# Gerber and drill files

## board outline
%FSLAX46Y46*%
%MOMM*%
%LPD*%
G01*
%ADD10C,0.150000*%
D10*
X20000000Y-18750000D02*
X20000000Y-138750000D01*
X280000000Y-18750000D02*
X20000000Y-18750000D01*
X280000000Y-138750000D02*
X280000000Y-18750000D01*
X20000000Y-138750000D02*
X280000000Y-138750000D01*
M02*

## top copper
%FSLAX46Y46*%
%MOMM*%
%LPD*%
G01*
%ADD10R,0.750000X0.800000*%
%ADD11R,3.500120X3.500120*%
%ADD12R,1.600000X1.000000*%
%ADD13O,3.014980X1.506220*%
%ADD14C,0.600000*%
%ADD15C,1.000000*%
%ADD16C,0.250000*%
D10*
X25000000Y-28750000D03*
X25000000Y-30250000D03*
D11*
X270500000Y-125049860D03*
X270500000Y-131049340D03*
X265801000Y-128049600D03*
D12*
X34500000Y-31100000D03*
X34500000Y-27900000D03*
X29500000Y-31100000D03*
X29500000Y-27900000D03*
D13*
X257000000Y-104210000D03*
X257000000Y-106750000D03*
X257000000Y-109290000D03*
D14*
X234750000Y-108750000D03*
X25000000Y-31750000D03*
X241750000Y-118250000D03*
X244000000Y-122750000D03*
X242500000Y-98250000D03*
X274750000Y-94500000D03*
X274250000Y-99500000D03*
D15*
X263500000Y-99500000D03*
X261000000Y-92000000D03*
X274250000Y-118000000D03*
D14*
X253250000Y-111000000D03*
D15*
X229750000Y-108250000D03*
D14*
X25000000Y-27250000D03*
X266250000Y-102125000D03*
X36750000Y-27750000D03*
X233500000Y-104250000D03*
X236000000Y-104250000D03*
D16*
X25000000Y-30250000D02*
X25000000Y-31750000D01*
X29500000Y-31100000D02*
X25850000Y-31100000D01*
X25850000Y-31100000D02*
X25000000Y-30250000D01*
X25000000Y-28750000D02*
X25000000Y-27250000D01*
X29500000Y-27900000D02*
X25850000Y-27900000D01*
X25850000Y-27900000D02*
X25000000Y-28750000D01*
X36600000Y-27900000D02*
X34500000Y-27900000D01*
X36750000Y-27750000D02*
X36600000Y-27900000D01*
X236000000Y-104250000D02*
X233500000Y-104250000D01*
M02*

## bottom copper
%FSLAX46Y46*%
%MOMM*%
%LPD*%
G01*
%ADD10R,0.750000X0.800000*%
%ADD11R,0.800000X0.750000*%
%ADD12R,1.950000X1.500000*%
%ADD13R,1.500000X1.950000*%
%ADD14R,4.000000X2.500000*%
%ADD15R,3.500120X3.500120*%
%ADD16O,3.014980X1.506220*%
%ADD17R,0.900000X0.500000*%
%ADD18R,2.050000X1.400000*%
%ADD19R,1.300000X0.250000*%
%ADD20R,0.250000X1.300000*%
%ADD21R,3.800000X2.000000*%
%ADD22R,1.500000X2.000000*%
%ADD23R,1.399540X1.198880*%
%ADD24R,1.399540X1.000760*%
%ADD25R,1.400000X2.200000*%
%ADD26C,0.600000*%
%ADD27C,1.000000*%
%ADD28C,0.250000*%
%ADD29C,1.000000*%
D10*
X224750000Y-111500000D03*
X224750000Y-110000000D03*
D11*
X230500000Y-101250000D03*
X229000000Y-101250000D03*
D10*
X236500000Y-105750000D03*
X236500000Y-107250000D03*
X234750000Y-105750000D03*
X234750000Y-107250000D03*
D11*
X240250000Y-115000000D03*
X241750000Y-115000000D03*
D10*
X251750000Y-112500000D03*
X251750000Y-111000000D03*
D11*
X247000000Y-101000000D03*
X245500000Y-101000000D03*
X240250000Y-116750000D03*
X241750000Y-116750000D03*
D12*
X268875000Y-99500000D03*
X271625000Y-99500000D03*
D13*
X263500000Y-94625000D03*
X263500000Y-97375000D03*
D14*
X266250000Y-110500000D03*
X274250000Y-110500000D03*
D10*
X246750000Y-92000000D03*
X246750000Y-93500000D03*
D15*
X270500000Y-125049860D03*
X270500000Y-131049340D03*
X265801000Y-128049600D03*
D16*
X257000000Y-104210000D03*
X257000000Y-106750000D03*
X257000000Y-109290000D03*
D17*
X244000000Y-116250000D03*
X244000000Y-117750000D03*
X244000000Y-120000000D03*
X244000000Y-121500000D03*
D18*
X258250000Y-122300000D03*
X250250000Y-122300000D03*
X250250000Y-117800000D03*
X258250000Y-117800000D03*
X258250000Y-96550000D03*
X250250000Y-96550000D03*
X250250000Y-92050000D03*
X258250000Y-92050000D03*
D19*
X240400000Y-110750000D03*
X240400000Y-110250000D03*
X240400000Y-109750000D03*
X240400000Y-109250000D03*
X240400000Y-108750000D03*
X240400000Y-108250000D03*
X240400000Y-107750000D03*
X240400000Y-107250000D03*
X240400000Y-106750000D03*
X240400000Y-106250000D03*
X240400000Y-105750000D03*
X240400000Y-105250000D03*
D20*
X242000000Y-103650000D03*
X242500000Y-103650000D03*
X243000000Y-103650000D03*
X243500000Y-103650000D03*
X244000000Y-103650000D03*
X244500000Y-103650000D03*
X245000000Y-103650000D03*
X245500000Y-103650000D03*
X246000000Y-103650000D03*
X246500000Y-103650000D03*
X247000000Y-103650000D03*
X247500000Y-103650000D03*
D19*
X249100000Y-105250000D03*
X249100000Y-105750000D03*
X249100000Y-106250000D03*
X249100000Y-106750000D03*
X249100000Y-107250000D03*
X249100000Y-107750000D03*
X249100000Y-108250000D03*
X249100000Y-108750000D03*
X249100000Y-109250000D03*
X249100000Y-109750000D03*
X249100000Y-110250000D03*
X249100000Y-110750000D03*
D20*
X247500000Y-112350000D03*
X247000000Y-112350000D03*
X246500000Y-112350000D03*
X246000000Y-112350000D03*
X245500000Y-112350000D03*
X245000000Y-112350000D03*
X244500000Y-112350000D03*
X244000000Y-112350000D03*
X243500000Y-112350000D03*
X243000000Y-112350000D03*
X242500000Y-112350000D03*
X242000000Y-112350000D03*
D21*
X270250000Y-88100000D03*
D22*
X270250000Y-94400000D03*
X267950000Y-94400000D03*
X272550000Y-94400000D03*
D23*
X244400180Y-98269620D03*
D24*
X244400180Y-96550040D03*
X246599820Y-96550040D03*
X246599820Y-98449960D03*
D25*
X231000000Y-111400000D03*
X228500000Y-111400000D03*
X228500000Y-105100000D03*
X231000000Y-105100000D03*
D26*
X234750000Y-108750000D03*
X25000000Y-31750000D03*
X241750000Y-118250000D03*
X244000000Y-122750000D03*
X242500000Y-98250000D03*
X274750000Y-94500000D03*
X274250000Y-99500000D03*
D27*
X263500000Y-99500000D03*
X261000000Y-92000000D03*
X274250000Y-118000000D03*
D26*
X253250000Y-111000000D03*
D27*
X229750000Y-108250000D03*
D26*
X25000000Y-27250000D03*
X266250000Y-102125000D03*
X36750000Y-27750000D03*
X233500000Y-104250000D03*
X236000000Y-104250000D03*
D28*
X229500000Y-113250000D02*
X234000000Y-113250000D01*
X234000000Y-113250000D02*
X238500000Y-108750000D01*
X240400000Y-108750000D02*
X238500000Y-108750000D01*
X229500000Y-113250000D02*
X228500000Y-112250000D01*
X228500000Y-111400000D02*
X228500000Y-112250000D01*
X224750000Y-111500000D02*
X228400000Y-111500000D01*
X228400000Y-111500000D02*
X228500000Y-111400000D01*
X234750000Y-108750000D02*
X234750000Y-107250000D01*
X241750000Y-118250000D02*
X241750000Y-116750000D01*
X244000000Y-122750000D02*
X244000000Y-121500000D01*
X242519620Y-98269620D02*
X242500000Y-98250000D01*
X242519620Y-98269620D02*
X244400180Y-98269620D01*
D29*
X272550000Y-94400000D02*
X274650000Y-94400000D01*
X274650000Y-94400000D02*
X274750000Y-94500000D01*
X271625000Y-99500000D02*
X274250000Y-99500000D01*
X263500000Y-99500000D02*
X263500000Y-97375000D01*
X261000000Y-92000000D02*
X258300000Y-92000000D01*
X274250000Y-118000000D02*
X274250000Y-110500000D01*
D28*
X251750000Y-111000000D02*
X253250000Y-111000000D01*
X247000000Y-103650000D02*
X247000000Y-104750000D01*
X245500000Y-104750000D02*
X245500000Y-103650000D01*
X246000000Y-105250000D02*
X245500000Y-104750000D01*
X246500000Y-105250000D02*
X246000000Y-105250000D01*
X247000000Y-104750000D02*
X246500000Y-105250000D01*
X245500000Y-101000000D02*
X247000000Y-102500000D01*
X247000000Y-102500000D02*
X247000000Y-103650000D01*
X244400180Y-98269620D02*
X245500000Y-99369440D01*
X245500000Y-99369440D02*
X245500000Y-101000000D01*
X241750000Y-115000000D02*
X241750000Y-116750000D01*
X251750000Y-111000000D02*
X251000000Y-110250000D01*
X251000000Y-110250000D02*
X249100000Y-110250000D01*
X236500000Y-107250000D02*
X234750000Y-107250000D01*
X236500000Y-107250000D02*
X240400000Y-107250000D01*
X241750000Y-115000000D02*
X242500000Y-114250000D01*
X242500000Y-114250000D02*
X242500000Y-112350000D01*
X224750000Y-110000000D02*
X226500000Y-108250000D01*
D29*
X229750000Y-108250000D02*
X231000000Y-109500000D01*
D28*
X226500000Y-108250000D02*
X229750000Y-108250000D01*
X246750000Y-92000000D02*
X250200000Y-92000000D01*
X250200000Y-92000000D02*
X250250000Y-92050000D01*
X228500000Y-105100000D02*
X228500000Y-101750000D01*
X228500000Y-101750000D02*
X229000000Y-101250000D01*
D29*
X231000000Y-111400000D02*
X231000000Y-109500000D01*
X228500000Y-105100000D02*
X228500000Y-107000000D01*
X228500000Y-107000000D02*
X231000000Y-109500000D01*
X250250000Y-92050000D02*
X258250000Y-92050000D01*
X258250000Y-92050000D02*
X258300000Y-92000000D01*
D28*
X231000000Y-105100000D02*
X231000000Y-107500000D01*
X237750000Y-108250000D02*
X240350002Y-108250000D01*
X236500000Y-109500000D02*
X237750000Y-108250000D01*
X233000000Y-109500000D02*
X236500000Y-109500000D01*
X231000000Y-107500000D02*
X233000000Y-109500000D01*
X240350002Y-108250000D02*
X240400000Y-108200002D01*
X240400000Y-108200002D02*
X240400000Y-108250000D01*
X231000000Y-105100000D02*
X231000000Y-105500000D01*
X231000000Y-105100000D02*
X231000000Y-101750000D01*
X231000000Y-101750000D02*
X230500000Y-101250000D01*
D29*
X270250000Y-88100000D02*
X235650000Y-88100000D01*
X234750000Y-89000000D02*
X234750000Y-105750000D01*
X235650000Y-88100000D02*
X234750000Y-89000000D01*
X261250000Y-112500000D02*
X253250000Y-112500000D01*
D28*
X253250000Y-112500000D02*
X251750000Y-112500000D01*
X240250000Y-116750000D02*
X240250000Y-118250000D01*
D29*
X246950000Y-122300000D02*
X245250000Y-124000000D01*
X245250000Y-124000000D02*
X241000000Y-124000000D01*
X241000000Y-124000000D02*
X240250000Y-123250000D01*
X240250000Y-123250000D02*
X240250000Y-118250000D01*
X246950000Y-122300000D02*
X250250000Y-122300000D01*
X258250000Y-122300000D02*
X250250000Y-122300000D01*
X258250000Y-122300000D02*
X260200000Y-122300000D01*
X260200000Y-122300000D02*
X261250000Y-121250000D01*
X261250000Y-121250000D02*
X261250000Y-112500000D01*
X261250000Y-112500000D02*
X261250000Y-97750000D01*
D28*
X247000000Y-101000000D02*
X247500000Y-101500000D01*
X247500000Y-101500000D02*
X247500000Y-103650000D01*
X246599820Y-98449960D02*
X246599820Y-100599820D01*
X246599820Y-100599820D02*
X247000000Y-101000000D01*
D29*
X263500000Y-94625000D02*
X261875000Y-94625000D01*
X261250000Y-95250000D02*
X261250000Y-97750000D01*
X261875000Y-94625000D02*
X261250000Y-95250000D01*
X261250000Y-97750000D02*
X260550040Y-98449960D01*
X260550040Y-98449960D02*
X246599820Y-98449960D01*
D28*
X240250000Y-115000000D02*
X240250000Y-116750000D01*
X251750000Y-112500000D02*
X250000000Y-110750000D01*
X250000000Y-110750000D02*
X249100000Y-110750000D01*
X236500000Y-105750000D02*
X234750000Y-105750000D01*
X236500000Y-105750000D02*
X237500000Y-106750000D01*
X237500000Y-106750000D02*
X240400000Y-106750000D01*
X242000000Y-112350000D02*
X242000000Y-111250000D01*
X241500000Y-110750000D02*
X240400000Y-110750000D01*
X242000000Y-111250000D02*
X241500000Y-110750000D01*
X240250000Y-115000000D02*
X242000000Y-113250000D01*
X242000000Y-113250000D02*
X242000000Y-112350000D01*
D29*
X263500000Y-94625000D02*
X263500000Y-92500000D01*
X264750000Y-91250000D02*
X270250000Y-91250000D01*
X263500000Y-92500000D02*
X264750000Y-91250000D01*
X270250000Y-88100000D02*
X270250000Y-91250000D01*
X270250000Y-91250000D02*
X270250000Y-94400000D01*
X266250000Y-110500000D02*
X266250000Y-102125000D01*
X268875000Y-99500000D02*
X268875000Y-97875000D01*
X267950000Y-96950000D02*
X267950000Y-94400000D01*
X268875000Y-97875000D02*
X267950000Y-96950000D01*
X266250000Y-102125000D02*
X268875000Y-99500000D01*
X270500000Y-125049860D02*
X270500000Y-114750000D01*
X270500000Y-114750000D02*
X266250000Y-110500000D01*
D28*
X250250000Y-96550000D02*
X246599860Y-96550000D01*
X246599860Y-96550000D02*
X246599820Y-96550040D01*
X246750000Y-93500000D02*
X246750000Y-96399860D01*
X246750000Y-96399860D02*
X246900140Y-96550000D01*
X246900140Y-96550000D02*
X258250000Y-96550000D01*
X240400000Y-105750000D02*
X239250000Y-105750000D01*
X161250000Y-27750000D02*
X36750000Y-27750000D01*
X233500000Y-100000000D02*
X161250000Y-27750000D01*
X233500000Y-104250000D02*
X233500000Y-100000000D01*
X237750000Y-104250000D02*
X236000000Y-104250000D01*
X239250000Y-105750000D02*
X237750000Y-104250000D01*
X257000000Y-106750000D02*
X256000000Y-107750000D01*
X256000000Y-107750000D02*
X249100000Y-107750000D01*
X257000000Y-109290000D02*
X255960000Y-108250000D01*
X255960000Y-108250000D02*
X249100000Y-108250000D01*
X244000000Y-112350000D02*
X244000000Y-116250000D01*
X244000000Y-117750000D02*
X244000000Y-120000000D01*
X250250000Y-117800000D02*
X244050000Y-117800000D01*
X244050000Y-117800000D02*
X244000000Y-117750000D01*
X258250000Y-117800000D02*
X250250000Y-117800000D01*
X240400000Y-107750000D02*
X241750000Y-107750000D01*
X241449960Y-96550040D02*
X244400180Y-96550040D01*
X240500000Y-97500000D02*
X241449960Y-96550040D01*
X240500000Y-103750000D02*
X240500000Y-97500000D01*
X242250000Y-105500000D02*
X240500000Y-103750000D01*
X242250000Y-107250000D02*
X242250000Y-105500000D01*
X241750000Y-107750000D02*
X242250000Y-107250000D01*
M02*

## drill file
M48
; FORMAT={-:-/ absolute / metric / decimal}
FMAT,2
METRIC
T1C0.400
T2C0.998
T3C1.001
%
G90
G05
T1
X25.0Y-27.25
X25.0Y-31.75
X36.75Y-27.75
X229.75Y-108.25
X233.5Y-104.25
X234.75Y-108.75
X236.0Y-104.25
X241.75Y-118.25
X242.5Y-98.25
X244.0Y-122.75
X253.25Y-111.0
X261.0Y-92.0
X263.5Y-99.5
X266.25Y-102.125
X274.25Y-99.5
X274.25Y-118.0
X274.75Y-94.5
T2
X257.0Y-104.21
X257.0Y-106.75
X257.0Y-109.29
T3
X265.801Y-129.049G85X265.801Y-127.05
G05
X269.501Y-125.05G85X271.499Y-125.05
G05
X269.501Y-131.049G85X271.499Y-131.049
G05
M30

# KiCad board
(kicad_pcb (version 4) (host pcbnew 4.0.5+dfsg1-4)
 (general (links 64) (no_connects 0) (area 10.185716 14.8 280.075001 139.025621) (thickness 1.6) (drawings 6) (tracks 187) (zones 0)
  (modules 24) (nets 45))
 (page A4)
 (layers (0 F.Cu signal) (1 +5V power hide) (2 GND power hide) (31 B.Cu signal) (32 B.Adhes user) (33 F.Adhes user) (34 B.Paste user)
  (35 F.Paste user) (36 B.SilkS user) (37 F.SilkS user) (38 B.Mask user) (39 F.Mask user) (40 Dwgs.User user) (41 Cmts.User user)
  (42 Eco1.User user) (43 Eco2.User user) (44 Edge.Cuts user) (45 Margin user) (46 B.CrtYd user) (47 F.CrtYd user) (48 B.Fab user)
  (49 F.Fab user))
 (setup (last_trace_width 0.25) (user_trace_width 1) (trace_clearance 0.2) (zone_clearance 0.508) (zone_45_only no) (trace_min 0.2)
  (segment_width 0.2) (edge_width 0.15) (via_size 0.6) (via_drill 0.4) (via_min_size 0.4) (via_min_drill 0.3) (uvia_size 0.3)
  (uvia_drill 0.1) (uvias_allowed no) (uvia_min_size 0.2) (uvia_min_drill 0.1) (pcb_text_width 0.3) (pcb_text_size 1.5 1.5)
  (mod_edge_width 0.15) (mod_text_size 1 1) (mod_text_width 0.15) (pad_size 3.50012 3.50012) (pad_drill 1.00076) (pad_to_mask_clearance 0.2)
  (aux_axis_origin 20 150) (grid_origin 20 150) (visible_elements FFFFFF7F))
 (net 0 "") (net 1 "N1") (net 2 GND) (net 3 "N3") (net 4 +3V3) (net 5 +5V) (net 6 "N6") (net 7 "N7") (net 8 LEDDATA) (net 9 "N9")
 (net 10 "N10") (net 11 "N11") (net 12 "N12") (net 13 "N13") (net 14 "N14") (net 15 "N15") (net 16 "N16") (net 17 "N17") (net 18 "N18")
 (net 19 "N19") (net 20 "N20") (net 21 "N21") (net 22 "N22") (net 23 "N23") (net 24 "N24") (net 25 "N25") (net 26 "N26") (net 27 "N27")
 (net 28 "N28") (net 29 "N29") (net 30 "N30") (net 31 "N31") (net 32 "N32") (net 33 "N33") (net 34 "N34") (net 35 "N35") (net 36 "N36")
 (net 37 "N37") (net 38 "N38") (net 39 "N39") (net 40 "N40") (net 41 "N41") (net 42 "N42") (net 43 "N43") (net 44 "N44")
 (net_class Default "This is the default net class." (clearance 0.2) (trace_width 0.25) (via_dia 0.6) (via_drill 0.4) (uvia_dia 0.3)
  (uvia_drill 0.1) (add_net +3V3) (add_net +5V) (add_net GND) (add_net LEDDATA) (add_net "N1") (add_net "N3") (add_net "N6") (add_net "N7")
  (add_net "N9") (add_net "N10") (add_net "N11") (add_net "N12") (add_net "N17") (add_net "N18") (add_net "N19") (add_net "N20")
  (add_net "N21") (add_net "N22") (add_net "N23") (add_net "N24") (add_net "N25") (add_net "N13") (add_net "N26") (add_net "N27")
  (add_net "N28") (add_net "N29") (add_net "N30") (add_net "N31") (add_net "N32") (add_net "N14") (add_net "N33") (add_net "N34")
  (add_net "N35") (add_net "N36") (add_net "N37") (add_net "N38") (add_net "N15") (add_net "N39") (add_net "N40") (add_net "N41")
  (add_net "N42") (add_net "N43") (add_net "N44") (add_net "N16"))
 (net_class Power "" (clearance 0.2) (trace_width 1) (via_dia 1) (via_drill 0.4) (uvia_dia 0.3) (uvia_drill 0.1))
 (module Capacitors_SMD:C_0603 (layer B.Cu) (at 224.75 110.75 90)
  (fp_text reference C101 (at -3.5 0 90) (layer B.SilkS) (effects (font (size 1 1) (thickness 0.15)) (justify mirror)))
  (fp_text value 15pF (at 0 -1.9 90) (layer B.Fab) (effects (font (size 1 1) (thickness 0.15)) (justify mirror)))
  (pad 1 smd rect (at -0.75 0 90) (size 0.8 0.75) (layers B.Cu B.Paste B.Mask) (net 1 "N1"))
  (pad 2 smd rect (at 0.75 0 90) (size 0.8 0.75) (layers B.Cu B.Paste B.Mask) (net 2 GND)))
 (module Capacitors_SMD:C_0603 (layer B.Cu) (at 229.75 101.25 180)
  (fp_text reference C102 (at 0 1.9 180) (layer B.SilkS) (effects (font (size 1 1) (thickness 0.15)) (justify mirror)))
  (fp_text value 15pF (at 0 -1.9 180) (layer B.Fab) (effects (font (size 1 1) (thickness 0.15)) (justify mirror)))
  (pad 1 smd rect (at -0.75 0 180) (size 0.8 0.75) (layers B.Cu B.Paste B.Mask) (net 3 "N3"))
  (pad 2 smd rect (at 0.75 0 180) (size 0.8 0.75) (layers B.Cu B.Paste B.Mask) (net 2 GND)))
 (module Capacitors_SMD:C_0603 (layer B.Cu) (at 236.5 106.5 270)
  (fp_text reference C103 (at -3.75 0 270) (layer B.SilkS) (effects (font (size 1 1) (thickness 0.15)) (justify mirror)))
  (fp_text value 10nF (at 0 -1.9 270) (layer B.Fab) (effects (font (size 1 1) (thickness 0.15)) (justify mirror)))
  (pad 1 smd rect (at -0.75 0 270) (size 0.8 0.75) (layers B.Cu B.Paste B.Mask) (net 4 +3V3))
  (pad 2 smd rect (at 0.75 0 270) (size 0.8 0.75) (layers B.Cu B.Paste B.Mask) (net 2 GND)))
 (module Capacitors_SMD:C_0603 (layer B.Cu) (at 234.75 106.5 270)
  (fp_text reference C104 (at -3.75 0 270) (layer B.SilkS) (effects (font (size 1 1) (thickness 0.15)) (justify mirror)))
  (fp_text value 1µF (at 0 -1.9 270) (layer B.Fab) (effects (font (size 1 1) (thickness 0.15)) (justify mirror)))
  (pad 1 smd rect (at -0.75 0 270) (size 0.8 0.75) (layers B.Cu B.Paste B.Mask) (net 4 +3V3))
  (pad 2 smd rect (at 0.75 0 270) (size 0.8 0.75) (layers B.Cu B.Paste B.Mask) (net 2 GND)))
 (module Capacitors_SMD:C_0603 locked (layer B.Cu) (at 241 115)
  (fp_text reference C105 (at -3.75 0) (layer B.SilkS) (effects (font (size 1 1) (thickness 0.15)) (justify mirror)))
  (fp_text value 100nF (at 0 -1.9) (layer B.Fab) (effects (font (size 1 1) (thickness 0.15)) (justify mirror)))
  (pad 1 smd rect (at -0.75 0) (size 0.8 0.75) (layers B.Cu B.Paste B.Mask) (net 4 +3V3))
  (pad 2 smd rect (at 0.75 0) (size 0.8 0.75) (layers B.Cu B.Paste B.Mask) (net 2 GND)))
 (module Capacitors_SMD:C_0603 (layer B.Cu) (at 251.75 111.75 90)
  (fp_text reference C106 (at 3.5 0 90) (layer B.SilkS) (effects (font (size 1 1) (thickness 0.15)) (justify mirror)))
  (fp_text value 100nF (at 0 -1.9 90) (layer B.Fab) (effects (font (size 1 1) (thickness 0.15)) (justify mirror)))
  (pad 1 smd rect (at -0.75 0 90) (size 0.8 0.75) (layers B.Cu B.Paste B.Mask) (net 4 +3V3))
  (pad 2 smd rect (at 0.75 0 90) (size 0.8 0.75) (layers B.Cu B.Paste B.Mask) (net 2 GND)))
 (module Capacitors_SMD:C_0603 (layer B.Cu) (at 246.25 101 180)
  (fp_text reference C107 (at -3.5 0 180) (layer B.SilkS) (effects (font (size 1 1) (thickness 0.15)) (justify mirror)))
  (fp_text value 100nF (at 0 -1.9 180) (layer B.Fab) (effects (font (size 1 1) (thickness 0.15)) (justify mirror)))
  (pad 1 smd rect (at -0.75 0 180) (size 0.8 0.75) (layers B.Cu B.Paste B.Mask) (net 4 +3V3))
  (pad 2 smd rect (at 0.75 0 180) (size 0.8 0.75) (layers B.Cu B.Paste B.Mask) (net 2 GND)))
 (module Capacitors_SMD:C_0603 (layer B.Cu) (at 241 116.75)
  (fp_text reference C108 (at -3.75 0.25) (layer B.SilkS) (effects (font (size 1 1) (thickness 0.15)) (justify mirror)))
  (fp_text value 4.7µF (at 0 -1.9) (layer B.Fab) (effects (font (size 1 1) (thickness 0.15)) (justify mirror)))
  (pad 1 smd rect (at -0.75 0) (size 0.8 0.75) (layers B.Cu B.Paste B.Mask) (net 4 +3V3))
  (pad 2 smd rect (at 0.75 0) (size 0.8 0.75) (layers B.Cu B.Paste B.Mask) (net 2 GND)))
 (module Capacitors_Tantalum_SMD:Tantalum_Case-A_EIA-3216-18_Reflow (layer B.Cu) (at 270.25 99.5)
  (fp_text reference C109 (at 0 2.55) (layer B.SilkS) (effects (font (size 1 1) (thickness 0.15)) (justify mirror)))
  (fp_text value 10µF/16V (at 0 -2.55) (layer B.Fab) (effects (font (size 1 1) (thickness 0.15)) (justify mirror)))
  (pad 1 smd rect (at -1.375 0) (size 1.95 1.5) (layers B.Cu B.Paste B.Mask) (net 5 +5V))
  (pad 2 smd rect (at 1.375 0) (size 1.95 1.5) (layers B.Cu B.Paste B.Mask) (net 2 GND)))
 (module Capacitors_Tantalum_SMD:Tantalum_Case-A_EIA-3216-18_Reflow (layer B.Cu) (at 263.5 96 270)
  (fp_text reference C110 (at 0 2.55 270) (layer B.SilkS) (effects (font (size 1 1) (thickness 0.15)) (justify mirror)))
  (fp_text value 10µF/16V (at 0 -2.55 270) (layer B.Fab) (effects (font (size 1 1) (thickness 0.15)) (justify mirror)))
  (pad 1 smd rect (at -1.375 0 270) (size 1.95 1.5) (layers B.Cu B.Paste B.Mask) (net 4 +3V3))
  (pad 2 smd rect (at 1.375 0 270) (size 1.95 1.5) (layers B.Cu B.Paste B.Mask) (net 2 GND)))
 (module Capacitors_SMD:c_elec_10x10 (layer B.Cu) (at 270.25 110.5)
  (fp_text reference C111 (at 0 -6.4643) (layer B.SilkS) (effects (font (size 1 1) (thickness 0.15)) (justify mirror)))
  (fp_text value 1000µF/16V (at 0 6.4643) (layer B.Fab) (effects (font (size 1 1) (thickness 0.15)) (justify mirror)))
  (pad 1 smd rect (at -4 0 180) (size 4 2.5) (layers B.Cu B.Paste B.Mask) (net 5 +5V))
  (pad 2 smd rect (at 4 0 180) (size 4 2.5) (layers B.Cu B.Paste B.Mask) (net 2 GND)))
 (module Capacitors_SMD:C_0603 (layer B.Cu) (at 246.75 92.75 270)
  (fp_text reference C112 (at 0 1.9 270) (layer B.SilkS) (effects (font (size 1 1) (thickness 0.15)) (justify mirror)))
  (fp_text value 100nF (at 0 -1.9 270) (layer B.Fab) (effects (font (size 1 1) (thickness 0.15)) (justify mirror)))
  (pad 1 smd rect (at -0.75 0 270) (size 0.8 0.75) (layers B.Cu B.Paste B.Mask) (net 2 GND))
  (pad 2 smd rect (at 0.75 0 270) (size 0.8 0.75) (layers B.Cu B.Paste B.Mask) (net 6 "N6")))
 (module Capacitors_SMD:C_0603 (layer F.Cu) (at 25 29.5 270)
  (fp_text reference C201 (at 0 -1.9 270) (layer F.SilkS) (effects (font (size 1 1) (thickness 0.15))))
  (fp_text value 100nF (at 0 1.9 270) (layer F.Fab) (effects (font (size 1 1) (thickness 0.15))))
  (pad 1 smd rect (at -0.75 0 270) (size 0.8 0.75) (layers F.Cu F.Paste F.Mask) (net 5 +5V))
  (pad 2 smd rect (at 0.75 0 270) (size 0.8 0.75) (layers F.Cu F.Paste F.Mask) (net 2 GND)))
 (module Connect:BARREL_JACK (layer B.Cu) (at 270.5 131.25 90)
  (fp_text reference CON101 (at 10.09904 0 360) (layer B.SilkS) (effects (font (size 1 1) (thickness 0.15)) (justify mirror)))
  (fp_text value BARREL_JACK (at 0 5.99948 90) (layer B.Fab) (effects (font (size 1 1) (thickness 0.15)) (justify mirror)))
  (pad 1 thru_hole rect (at 6.20014 0 90) (size 3.50012 3.50012) (drill oval 1.00076 2.99974) (layers *.Cu *.Mask) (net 5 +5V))
  (pad 2 thru_hole rect (at 0.20066 0 90) (size 3.50012 3.50012) (drill oval 1.00076 2.99974) (layers *.Cu *.Mask) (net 2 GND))
  (pad 3 thru_hole rect (at 3.2004 -4.699 90) (size 3.50012 3.50012) (drill oval 2.99974 1.00076) (layers *.Cu *.Mask) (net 2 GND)))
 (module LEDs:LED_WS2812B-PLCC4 (layer F.Cu) (at 32 29.5)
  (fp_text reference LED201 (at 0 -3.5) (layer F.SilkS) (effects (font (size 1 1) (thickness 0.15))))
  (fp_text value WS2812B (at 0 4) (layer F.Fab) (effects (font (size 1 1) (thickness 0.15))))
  (pad 3 smd rect (at 2.5 1.6) (size 1.6 1) (layers F.Cu F.Paste F.Mask) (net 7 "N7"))
  (pad 4 smd rect (at 2.5 -1.6) (size 1.6 1) (layers F.Cu F.Paste F.Mask) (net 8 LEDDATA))
  (pad 2 smd rect (at -2.5 1.6) (size 1.6 1) (layers F.Cu F.Paste F.Mask) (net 2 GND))
  (pad 1 smd rect (at -2.5 -1.6) (size 1.6 1) (layers F.Cu F.Paste F.Mask) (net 5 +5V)))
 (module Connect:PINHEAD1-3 (layer B.Cu) (at 257 106.75 270)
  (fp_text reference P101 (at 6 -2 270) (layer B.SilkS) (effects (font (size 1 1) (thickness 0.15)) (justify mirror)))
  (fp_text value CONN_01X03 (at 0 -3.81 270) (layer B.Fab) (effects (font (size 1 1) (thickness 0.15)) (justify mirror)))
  (pad 1 thru_hole oval (at -2.54 0 270) (size 1.50622 3.01498) (drill 0.99822) (layers *.Cu *.Mask) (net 2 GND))
  (pad 2 thru_hole oval (at 0 0 270) (size 1.50622 3.01498) (drill 0.99822) (layers *.Cu *.Mask) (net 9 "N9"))
  (pad 3 thru_hole oval (at 2.54 0 270) (size 1.50622 3.01498) (drill 0.99822) (layers *.Cu *.Mask) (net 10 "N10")))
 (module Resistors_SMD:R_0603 (layer B.Cu) (at 244 117 270)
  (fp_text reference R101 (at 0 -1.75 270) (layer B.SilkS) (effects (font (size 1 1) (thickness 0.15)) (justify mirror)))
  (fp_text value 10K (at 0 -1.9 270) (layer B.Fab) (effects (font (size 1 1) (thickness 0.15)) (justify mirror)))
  (pad 1 smd rect (at -0.75 0 270) (size 0.5 0.9) (layers B.Cu B.Paste B.Mask) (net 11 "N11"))
  (pad 2 smd rect (at 0.75 0 270) (size 0.5 0.9) (layers B.Cu B.Paste B.Mask) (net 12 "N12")))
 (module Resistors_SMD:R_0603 (layer B.Cu) (at 244 120.75 270)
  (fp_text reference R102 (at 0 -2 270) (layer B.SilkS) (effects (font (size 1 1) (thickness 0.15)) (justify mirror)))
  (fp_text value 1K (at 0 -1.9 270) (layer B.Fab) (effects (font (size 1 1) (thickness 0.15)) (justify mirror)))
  (pad 1 smd rect (at -0.75 0 270) (size 0.5 0.9) (layers B.Cu B.Paste B.Mask) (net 12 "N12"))
  (pad 2 smd rect (at 0.75 0 270) (size 0.5 0.9) (layers B.Cu B.Paste B.Mask) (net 2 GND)))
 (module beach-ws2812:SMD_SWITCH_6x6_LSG (layer B.Cu) (at 249.25 123)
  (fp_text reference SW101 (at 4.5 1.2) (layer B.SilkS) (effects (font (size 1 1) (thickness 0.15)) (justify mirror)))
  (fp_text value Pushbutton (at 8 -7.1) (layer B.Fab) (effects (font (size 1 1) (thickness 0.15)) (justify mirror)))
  (pad 2 smd rect (at 9 -0.7) (size 2.05 1.4) (layers B.Cu B.Paste B.Mask) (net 4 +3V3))
  (pad 1 smd rect (at 1 -0.7) (size 2.05 1.4) (layers B.Cu B.Paste B.Mask) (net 4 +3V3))
  (pad 3 smd rect (at 1 -5.2) (size 2.05 1.4) (layers B.Cu B.Paste B.Mask) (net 12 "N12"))
  (pad 4 smd rect (at 9 -5.2) (size 2.05 1.4) (layers B.Cu B.Paste B.Mask) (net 12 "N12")))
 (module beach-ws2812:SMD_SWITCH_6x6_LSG (layer B.Cu) (at 249.25 97.25)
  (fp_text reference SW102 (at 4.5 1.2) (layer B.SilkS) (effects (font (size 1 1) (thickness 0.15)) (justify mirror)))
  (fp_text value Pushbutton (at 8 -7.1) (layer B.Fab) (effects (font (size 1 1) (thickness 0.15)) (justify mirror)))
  (pad 2 smd rect (at 9 -0.7) (size 2.05 1.4) (layers B.Cu B.Paste B.Mask) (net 6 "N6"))
  (pad 1 smd rect (at 1 -0.7) (size 2.05 1.4) (layers B.Cu B.Paste B.Mask) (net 6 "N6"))
  (pad 3 smd rect (at 1 -5.2) (size 2.05 1.4) (layers B.Cu B.Paste B.Mask) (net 2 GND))
  (pad 4 smd rect (at 9 -5.2) (size 2.05 1.4) (layers B.Cu B.Paste B.Mask) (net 2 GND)))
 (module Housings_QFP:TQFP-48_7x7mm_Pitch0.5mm (layer B.Cu) (at 244.75 108)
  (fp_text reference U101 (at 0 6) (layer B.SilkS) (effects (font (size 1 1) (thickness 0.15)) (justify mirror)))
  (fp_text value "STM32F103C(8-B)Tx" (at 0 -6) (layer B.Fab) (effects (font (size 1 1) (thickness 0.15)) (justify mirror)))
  (pad 1 smd rect (at -4.35 2.75) (size 1.3 0.25) (layers B.Cu B.Paste B.Mask) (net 4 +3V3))
  (pad 2 smd rect (at -4.35 2.25) (size 1.3 0.25) (layers B.Cu B.Paste B.Mask) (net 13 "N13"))
  (pad 3 smd rect (at -4.35 1.75) (size 1.3 0.25) (layers B.Cu B.Paste B.Mask) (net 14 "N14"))
  (pad 4 smd rect (at -4.35 1.25) (size 1.3 0.25) (layers B.Cu B.Paste B.Mask) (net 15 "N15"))
  (pad 5 smd rect (at -4.35 0.75) (size 1.3 0.25) (layers B.Cu B.Paste B.Mask) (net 1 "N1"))
  (pad 6 smd rect (at -4.35 0.25) (size 1.3 0.25) (layers B.Cu B.Paste B.Mask) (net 3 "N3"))
  (pad 7 smd rect (at -4.35 -0.25) (size 1.3 0.25) (layers B.Cu B.Paste B.Mask) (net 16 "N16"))
  (pad 8 smd rect (at -4.35 -0.75) (size 1.3 0.25) (layers B.Cu B.Paste B.Mask) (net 2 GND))
  (pad 9 smd rect (at -4.35 -1.25) (size 1.3 0.25) (layers B.Cu B.Paste B.Mask) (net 4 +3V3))
  (pad 10 smd rect (at -4.35 -1.75) (size 1.3 0.25) (layers B.Cu B.Paste B.Mask) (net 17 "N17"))
  (pad 11 smd rect (at -4.35 -2.25) (size 1.3 0.25) (layers B.Cu B.Paste B.Mask) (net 8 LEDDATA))
  (pad 12 smd rect (at -4.35 -2.75) (size 1.3 0.25) (layers B.Cu B.Paste B.Mask) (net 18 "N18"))
  (pad 13 smd rect (at -2.75 -4.35 270) (size 1.3 0.25) (layers B.Cu B.Paste B.Mask) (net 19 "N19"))
  (pad 14 smd rect (at -2.25 -4.35 270) (size 1.3 0.25) (layers B.Cu B.Paste B.Mask) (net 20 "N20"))
  (pad 15 smd rect (at -1.75 -4.35 270) (size 1.3 0.25) (layers B.Cu B.Paste B.Mask) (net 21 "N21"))
  (pad 16 smd rect (at -1.25 -4.35 270) (size 1.3 0.25) (layers B.Cu B.Paste B.Mask) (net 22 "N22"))
  (pad 17 smd rect (at -0.75 -4.35 270) (size 1.3 0.25) (layers B.Cu B.Paste B.Mask) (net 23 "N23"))
  (pad 18 smd rect (at -0.25 -4.35 270) (size 1.3 0.25) (layers B.Cu B.Paste B.Mask) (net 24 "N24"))
  (pad 19 smd rect (at 0.25 -4.35 270) (size 1.3 0.25) (layers B.Cu B.Paste B.Mask) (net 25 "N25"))
  (pad 20 smd rect (at 0.75 -4.35 270) (size 1.3 0.25) (layers B.Cu B.Paste B.Mask) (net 2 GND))
  (pad 21 smd rect (at 1.25 -4.35 270) (size 1.3 0.25) (layers B.Cu B.Paste B.Mask) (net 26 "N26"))
  (pad 22 smd rect (at 1.75 -4.35 270) (size 1.3 0.25) (layers B.Cu B.Paste B.Mask) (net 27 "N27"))
  (pad 23 smd rect (at 2.25 -4.35 270) (size 1.3 0.25) (layers B.Cu B.Paste B.Mask) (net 2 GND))
  (pad 24 smd rect (at 2.75 -4.35 270) (size 1.3 0.25) (layers B.Cu B.Paste B.Mask) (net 4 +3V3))
  (pad 25 smd rect (at 4.35 -2.75) (size 1.3 0.25) (layers B.Cu B.Paste B.Mask) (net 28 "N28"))
  (pad 26 smd rect (at 4.35 -2.25) (size 1.3 0.25) (layers B.Cu B.Paste B.Mask) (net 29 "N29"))
  (pad 27 smd rect (at 4.35 -1.75) (size 1.3 0.25) (layers B.Cu B.Paste B.Mask) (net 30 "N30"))
  (pad 28 smd rect (at 4.35 -1.25) (size 1.3 0.25) (layers B.Cu B.Paste B.Mask) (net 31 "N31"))
  (pad 29 smd rect (at 4.35 -0.75) (size 1.3 0.25) (layers B.Cu B.Paste B.Mask) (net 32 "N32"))
  (pad 30 smd rect (at 4.35 -0.25) (size 1.3 0.25) (layers B.Cu B.Paste B.Mask) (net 9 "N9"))
  (pad 31 smd rect (at 4.35 0.25) (size 1.3 0.25) (layers B.Cu B.Paste B.Mask) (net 10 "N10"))
  (pad 32 smd rect (at 4.35 0.75) (size 1.3 0.25) (layers B.Cu B.Paste B.Mask) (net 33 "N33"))
  (pad 33 smd rect (at 4.35 1.25) (size 1.3 0.25) (layers B.Cu B.Paste B.Mask) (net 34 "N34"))
  (pad 34 smd rect (at 4.35 1.75) (size 1.3 0.25) (layers B.Cu B.Paste B.Mask) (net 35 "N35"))
  (pad 35 smd rect (at 4.35 2.25) (size 1.3 0.25) (layers B.Cu B.Paste B.Mask) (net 2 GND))
  (pad 36 smd rect (at 4.35 2.75) (size 1.3 0.25) (layers B.Cu B.Paste B.Mask) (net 4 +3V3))
  (pad 37 smd rect (at 2.75 4.35 270) (size 1.3 0.25) (layers B.Cu B.Paste B.Mask) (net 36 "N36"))
  (pad 38 smd rect (at 2.25 4.35 270) (size 1.3 0.25) (layers B.Cu B.Paste B.Mask) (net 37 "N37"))
  (pad 39 smd rect (at 1.75 4.35 270) (size 1.3 0.25) (layers B.Cu B.Paste B.Mask) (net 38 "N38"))
  (pad 40 smd rect (at 1.25 4.35 270) (size 1.3 0.25) (layers B.Cu B.Paste B.Mask) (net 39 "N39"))
  (pad 41 smd rect (at 0.75 4.35 270) (size 1.3 0.25) (layers B.Cu B.Paste B.Mask) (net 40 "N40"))
  (pad 42 smd rect (at 0.25 4.35 270) (size 1.3 0.25) (layers B.Cu B.Paste B.Mask) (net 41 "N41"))
  (pad 43 smd rect (at -0.25 4.35 270) (size 1.3 0.25) (layers B.Cu B.Paste B.Mask) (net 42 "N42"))
  (pad 44 smd rect (at -0.75 4.35 270) (size 1.3 0.25) (layers B.Cu B.Paste B.Mask) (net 11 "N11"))
  (pad 45 smd rect (at -1.25 4.35 270) (size 1.3 0.25) (layers B.Cu B.Paste B.Mask) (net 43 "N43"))
  (pad 46 smd rect (at -1.75 4.35 270) (size 1.3 0.25) (layers B.Cu B.Paste B.Mask) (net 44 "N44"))
  (pad 47 smd rect (at -2.25 4.35 270) (size 1.3 0.25) (layers B.Cu B.Paste B.Mask) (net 2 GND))
  (pad 48 smd rect (at -2.75 4.35 270) (size 1.3 0.25) (layers B.Cu B.Paste B.Mask) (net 4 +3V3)))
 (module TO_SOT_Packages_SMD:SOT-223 (layer B.Cu) (at 270.25 91.25 90)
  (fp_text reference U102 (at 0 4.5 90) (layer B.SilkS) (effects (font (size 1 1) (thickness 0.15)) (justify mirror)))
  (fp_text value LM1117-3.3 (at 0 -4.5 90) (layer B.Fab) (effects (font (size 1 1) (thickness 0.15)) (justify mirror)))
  (pad 4 smd rect (at 3.15 0 90) (size 2 3.8) (layers B.Cu B.Paste B.Mask) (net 4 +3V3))
  (pad 2 smd rect (at -3.15 0 90) (size 2 1.5) (layers B.Cu B.Paste B.Mask) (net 4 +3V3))
  (pad 3 smd rect (at -3.15 -2.3 90) (size 2 1.5) (layers B.Cu B.Paste B.Mask) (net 5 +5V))
  (pad 1 smd rect (at -3.15 2.3 90) (size 2 1.5) (layers B.Cu B.Paste B.Mask) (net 2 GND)))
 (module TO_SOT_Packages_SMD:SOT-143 (layer B.Cu) (at 245.5 97.5 90)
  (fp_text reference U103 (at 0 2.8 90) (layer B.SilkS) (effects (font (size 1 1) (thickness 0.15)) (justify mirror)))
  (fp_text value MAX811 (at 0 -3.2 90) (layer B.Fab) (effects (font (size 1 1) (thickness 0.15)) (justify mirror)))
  (pad 1 smd rect (at -0.76962 -1.09982 90) (size 1.19888 1.39954) (layers B.Cu B.Paste B.Mask) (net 2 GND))
  (pad 2 smd rect (at 0.94996 -1.09982 90) (size 1.00076 1.39954) (layers B.Cu B.Paste B.Mask) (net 16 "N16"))
  (pad 3 smd rect (at 0.94996 1.09982 90) (size 1.00076 1.39954) (layers B.Cu B.Paste B.Mask) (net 6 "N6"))
  (pad 4 smd rect (at -0.94996 1.09982 90) (size 1.00076 1.39954) (layers B.Cu B.Paste B.Mask) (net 4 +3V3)))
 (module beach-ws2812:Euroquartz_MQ (layer B.Cu) (at 229.75 108.25 90)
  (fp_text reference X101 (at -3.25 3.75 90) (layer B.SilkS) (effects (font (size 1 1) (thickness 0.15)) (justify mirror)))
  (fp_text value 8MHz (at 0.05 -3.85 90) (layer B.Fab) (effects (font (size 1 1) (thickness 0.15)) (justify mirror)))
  (pad 4 smd rect (at -3.15 1.25 90) (size 2.2 1.4) (layers B.Cu B.Paste B.Mask) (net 2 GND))
  (pad 1 smd rect (at -3.15 -1.25 90) (size 2.2 1.4) (layers B.Cu B.Paste B.Mask) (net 1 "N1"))
  (pad 2 smd rect (at 3.15 -1.25 90) (size 2.2 1.4) (layers B.Cu B.Paste B.Mask) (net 2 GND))
  (pad 3 smd rect (at 3.15 1.25 90) (size 2.2 1.4) (layers B.Cu B.Paste B.Mask) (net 3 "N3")))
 (gr_line (start 20 18.75) (end 20 138.75) (angle 90) (layer Edge.Cuts) (width 0.15))
 (gr_line (start 280 18.75) (end 20 18.75) (angle 90) (layer Edge.Cuts) (width 0.15))
 (gr_line (start 280 138.75) (end 280 18.75) (angle 90) (layer Edge.Cuts) (width 0.15))
 (gr_line (start 20 138.75) (end 280 138.75) (angle 90) (layer Edge.Cuts) (width 0.15))
 (segment (start 229.5 113.25) (end 234 113.25) (width 0.25) (layer B.Cu) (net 1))
 (segment (start 234 113.25) (end 238.5 108.75) (width 0.25) (layer B.Cu) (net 1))
 (segment (start 240.4 108.75) (end 238.5 108.75) (width 0.25) (layer B.Cu) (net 1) (status 10))
 (segment (start 229.5 113.25) (end 228.5 112.25) (width 0.25) (layer B.Cu) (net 1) (status 20))
 (segment (start 228.5 111.4) (end 228.5 112.25) (width 0.25) (layer B.Cu) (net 1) (status 30))
 (segment (start 224.75 111.5) (end 228.4 111.5) (width 0.25) (layer B.Cu) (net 1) (status 30))
 (segment (start 228.4 111.5) (end 228.5 111.4) (width 0.25) (layer B.Cu) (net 1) (status 30))
 (segment (start 235.5 108.75) (end 234.75 108.75) (width 0.25) (layer GND) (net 2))
 (via (at 234.75 108.75) (size 0.6) (drill 0.4) (layers F.Cu B.Cu) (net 2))
 (segment (start 234.75 108.75) (end 234.75 107.25) (width 0.25) (layer B.Cu) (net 2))
 (segment (start 25 30.25) (end 25 31.75) (width 0.25) (layer F.Cu) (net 2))
 (segment (start 25 31.75) (end 26 31.75) (width 0.25) (layer GND) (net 2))
 (via (at 25 31.75) (size 0.6) (drill 0.4) (layers F.Cu B.Cu) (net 2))
 (segment (start 29.5 31.1) (end 25.85 31.1) (width 0.25) (layer F.Cu) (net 2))
 (segment (start 25.85 31.1) (end 25 30.25) (width 0.25) (layer F.Cu) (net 2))
 (segment (start 241.75 119.5) (end 241.75 118.25) (width 1) (layer GND) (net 2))
 (via (at 241.75 118.25) (size 0.6) (drill 0.4) (layers F.Cu B.Cu) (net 2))
 (segment (start 241.75 118.25) (end 241.75 116.75) (width 0.25) (layer B.Cu) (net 2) (status 20))
 (segment (start 242.75 122.75) (end 244 122.75) (width 1) (layer GND) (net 2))
 (via (at 244 122.75) (size 0.6) (drill 0.4) (layers F.Cu B.Cu) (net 2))
 (segment (start 244 122.75) (end 244 121.5) (width 0.25) (layer B.Cu) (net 2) (status 20))
 (segment (start 241.25 98.25) (end 242.5 98.25) (width 1) (layer GND) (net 2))
 (segment (start 242.51962 98.26962) (end 242.5 98.25) (width 0.25) (layer B.Cu) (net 2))
 (via (at 242.5 98.25) (size 0.6) (drill 0.4) (layers F.Cu B.Cu) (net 2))
 (segment (start 242.51962 98.26962) (end 244.40018 98.26962) (width 0.25) (layer B.Cu) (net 2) (status 20))
 (segment (start 272.55 94.4) (end 274.65 94.4) (width 1) (layer B.Cu) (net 2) (status 10))
 (segment (start 274.75 94.5) (end 276 94.5) (width 1) (layer GND) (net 2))
 (via (at 274.75 94.5) (size 0.6) (drill 0.4) (layers F.Cu B.Cu) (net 2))
 (segment (start 274.65 94.4) (end 274.75 94.5) (width 1) (layer B.Cu) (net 2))
 (segment (start 271.625 99.5) (end 274.25 99.5) (width 1) (layer B.Cu) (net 2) (status 10))
 (segment (start 274.25 99.5) (end 275.75 99.5) (width 1) (layer GND) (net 2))
 (via (at 274.25 99.5) (size 0.6) (drill 0.4) (layers F.Cu B.Cu) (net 2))
 (segment (start 263.5 101.25) (end 263.5 99.5) (width 1) (layer GND) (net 2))
 (via (at 263.5 99.5) (size 1) (drill 0.4) (layers F.Cu B.Cu) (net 2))
 (segment (start 263.5 99.5) (end 263.5 97.375) (width 1) (layer B.Cu) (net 2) (status 20))
 (segment (start 261 88.75) (end 261 92) (width 1) (layer GND) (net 2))
 (via (at 261 92) (size 1) (drill 0.4) (layers F.Cu B.Cu) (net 2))
 (segment (start 261 92) (end 258.3 92) (width 1) (layer B.Cu) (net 2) (status 20))
 (segment (start 265.801 128.0496) (end 268.2004 128.0496) (width 1) (layer GND) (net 2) (status 10))
 (segment (start 268.2004 128.0496) (end 268.25 128) (width 1) (layer GND) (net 2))
 (segment (start 265.801 128.0496) (end 265.801 125.301) (width 1) (layer GND) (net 2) (status 10))
 (segment (start 265.801 125.301) (end 265.75 125.25) (width 1) (layer GND) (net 2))
 (segment (start 265.801 128.0496) (end 265.801 131.949) (width 1) (layer GND) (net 2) (status 10))
 (segment (start 265.801 131.949) (end 265.75 132) (width 1) (layer GND) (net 2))
 (segment (start 265.801 128.0496) (end 263.0496 128.0496) (width 1) (layer GND) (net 2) (status 10))
 (segment (start 263.0496 128.0496) (end 263 128) (width 1) (layer GND) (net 2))
 (segment (start 270.5 131.04934) (end 270.5 128.25) (width 1) (layer GND) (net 2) (status 10))
 (segment (start 270.5 131.04934) (end 270.5 133.5) (width 1) (layer GND) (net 2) (status 10))
 (segment (start 270.5 131.04934) (end 270.5 133.5) (width 0.25) (layer GND) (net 2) (status 10))
 (segment (start 270.5 131.04934) (end 267.54934 131.04934) (width 1) (layer GND) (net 2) (status 10))
 (segment (start 267.54934 131.04934) (end 267.5 131) (width 1) (layer GND) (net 2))
 (segment (start 270.5 131.04934) (end 273.45066 131.04934) (width 1) (layer GND) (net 2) (status 10))
 (segment (start 273.45066 131.04934) (end 273.5 131) (width 1) (layer GND) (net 2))
 (segment (start 275.5 118) (end 274.25 118) (width 1) (layer GND) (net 2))
 (via (at 274.25 118) (size 1) (drill 0.4) (layers F.Cu B.Cu) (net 2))
 (segment (start 274.25 118) (end 274.25 110.5) (width 1) (layer B.Cu) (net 2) (status 20))
 (segment (start 251.75 111) (end 253.25 111) (width 0.25) (layer B.Cu) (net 2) (status 10))
 (via (at 253.25 111) (size 0.6) (drill 0.4) (layers F.Cu B.Cu) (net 2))
 (segment (start 247 103.65) (end 247 104.75) (width 0.25) (layer B.Cu) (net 2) (status 10))
 (segment (start 245.5 104.75) (end 245.5 103.65) (width 0.25) (layer B.Cu) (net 2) (status 20))
 (segment (start 246 105.25) (end 245.5 104.75) (width 0.25) (layer B.Cu) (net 2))
 (segment (start 246.5 105.25) (end 246 105.25) (width 0.25) (layer B.Cu) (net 2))
 (segment (start 247 104.75) (end 246.5 105.25) (width 0.25) (layer B.Cu) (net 2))
 (segment (start 245.5 101) (end 247 102.5) (width 0.25) (layer B.Cu) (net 2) (status 10))
 (segment (start 247 102.5) (end 247 103.65) (width 0.25) (layer B.Cu) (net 2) (status 20))
 (segment (start 244.40018 98.26962) (end 245.5 99.36944) (width 0.25) (layer B.Cu) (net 2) (status 10))
 (segment (start 245.5 99.36944) (end 245.5 101) (width 0.25) (layer B.Cu) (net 2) (status 20))
 (segment (start 241.75 115) (end 241.75 116.75) (width 0.25) (layer B.Cu) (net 2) (status 30))
 (segment (start 251.75 111) (end 251 110.25) (width 0.25) (layer B.Cu) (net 2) (status 10))
 (segment (start 251 110.25) (end 249.1 110.25) (width 0.25) (layer B.Cu) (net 2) (status 20))
 (segment (start 236.5 107.25) (end 234.75 107.25) (width 0.25) (layer B.Cu) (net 2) (status 30))
 (segment (start 236.5 107.25) (end 240.4 107.25) (width 0.25) (layer B.Cu) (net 2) (status 30))
 (segment (start 241.75 115) (end 242.5 114.25) (width 0.25) (layer B.Cu) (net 2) (status 10))
 (segment (start 242.5 114.25) (end 242.5 112.35) (width 0.25) (layer B.Cu) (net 2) (status 20))
 (segment (start 224.75 110) (end 226.5 108.25) (width 0.25) (layer B.Cu) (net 2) (status 10))
 (via (at 229.75 108.25) (size 1) (drill 0.4) (layers F.Cu B.Cu) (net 2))
 (segment (start 229.75 108.25) (end 231 109.5) (width 1) (layer B.Cu) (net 2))
 (segment (start 226.5 108.25) (end 229.75 108.25) (width 0.25) (layer B.Cu) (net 2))
 (segment (start 246.75 92) (end 250.2 92) (width 0.25) (layer B.Cu) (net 2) (status 30))
 (segment (start 250.2 92) (end 250.25 92.05) (width 0.25) (layer B.Cu) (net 2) (status 30))
 (segment (start 228.5 105.1) (end 228.5 101.75) (width 0.25) (layer B.Cu) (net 2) (status 10))
 (segment (start 228.5 101.75) (end 229 101.25) (width 0.25) (layer B.Cu) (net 2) (status 20))
 (segment (start 231 111.4) (end 231 109.5) (width 1) (layer B.Cu) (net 2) (status 10))
 (segment (start 228.5 105.1) (end 228.5 107) (width 1) (layer B.Cu) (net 2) (status 10))
 (segment (start 228.5 107) (end 231 109.5) (width 1) (layer B.Cu) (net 2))
 (segment (start 250.25 92.05) (end 258.25 92.05) (width 1) (layer B.Cu) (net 2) (status 30))
 (segment (start 258.25 92.05) (end 258.3 92) (width 1) (layer B.Cu) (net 2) (status 30))
 (segment (start 265.801 128.0496) (end 263.2996 128.0496) (width 0.25) (layer GND) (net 2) (status 10))
 (segment (start 263.2996 128.0496) (end 263.25 128) (width 0.25) (layer GND) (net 2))
 (segment (start 231 105.1) (end 231 107.5) (width 0.25) (layer B.Cu) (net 3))
 (segment (start 237.75 108.25) (end 240.350002 108.25) (width 0.25) (layer B.Cu) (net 3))
 (segment (start 236.5 109.5) (end 237.75 108.25) (width 0.25) (layer B.Cu) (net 3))
 (segment (start 233 109.5) (end 236.5 109.5) (width 0.25) (layer B.Cu) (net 3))
 (segment (start 231 107.5) (end 233 109.5) (width 0.25) (layer B.Cu) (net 3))
 (segment (start 240.350002 108.25) (end 240.4 108.200002) (width 0.25) (layer B.Cu) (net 3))
 (segment (start 240.4 108.200002) (end 240.4 108.25) (width 0.25) (layer B.Cu) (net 3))
 (segment (start 231 105.1) (end 231 105.5) (width 0.25) (layer B.Cu) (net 3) (status 30))
 (segment (start 231 105.1) (end 231 101.75) (width 0.25) (layer B.Cu) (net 3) (status 10))
 (segment (start 231 101.75) (end 230.5 101.25) (width 0.25) (layer B.Cu) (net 3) (status 20))
 (segment (start 270.25 88.1) (end 235.65 88.1) (width 1) (layer B.Cu) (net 4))
 (segment (start 234.75 89) (end 234.75 105.75) (width 1) (layer B.Cu) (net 4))
 (segment (start 235.65 88.1) (end 234.75 89) (width 1) (layer B.Cu) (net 4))
 (segment (start 261.25 112.5) (end 253.25 112.5) (width 1) (layer B.Cu) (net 4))
 (segment (start 253.25 112.5) (end 251.75 112.5) (width 0.25) (layer B.Cu) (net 4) (status 20))
 (segment (start 240.25 116.75) (end 240.25 118.25) (width 0.25) (layer B.Cu) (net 4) (status 10))
 (segment (start 246.95 122.3) (end 245.25 124) (width 1) (layer B.Cu) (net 4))
 (segment (start 245.25 124) (end 241 124) (width 1) (layer B.Cu) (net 4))
 (segment (start 241 124) (end 240.25 123.25) (width 1) (layer B.Cu) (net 4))
 (segment (start 240.25 123.25) (end 240.25 118.25) (width 1) (layer B.Cu) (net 4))
 (segment (start 246.95 122.3) (end 250.25 122.3) (width 1) (layer B.Cu) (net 4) (status 20))
 (segment (start 258.25 122.3) (end 250.25 122.3) (width 1) (layer B.Cu) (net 4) (status 30))
 (segment (start 258.25 122.3) (end 260.2 122.3) (width 1) (layer B.Cu) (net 4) (status 10))
 (segment (start 260.2 122.3) (end 261.25 121.25) (width 1) (layer B.Cu) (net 4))
 (segment (start 261.25 121.25) (end 261.25 112.5) (width 1) (layer B.Cu) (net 4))
 (segment (start 261.25 112.5) (end 261.25 97.75) (width 1) (layer B.Cu) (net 4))
 (segment (start 247 101) (end 247.5 101.5) (width 0.25) (layer B.Cu) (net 4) (status 10))
 (segment (start 247.5 101.5) (end 247.5 103.65) (width 0.25) (layer B.Cu) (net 4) (status 20))
 (segment (start 246.59982 98.44996) (end 246.59982 100.59982) (width 0.25) (layer B.Cu) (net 4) (status 10))
 (segment (start 246.59982 100.59982) (end 247 101) (width 0.25) (layer B.Cu) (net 4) (status 20))
 (segment (start 263.5 94.625) (end 261.875 94.625) (width 1) (layer B.Cu) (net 4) (status 10))
 (segment (start 261.25 95.25) (end 261.25 97.75) (width 1) (layer B.Cu) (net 4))
 (segment (start 261.875 94.625) (end 261.25 95.25) (width 1) (layer B.Cu) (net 4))
 (segment (start 261.25 97.75) (end 260.55004 98.44996) (width 1) (layer B.Cu) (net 4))
 (segment (start 260.55004 98.44996) (end 246.59982 98.44996) (width 1) (layer B.Cu) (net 4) (status 20))
 (segment (start 240.25 115) (end 240.25 116.75) (width 0.25) (layer B.Cu) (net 4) (status 30))
 (segment (start 251.75 112.5) (end 250 110.75) (width 0.25) (layer B.Cu) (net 4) (status 10))
 (segment (start 250 110.75) (end 249.1 110.75) (width 0.25) (layer B.Cu) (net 4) (status 20))
 (segment (start 236.5 105.75) (end 234.75 105.75) (width 0.25) (layer B.Cu) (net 4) (status 30))
 (segment (start 236.5 105.75) (end 237.5 106.75) (width 0.25) (layer B.Cu) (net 4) (status 10))
 (segment (start 237.5 106.75) (end 240.4 106.75) (width 0.25) (layer B.Cu) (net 4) (status 20))
 (segment (start 242 112.35) (end 242 111.25) (width 0.25) (layer B.Cu) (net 4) (status 10))
 (segment (start 241.5 110.75) (end 240.4 110.75) (width 0.25) (layer B.Cu) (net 4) (status 20))
 (segment (start 242 111.25) (end 241.5 110.75) (width 0.25) (layer B.Cu) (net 4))
 (segment (start 240.25 115) (end 242 113.25) (width 0.25) (layer B.Cu) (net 4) (status 10))
 (segment (start 242 113.25) (end 242 112.35) (width 0.25) (layer B.Cu) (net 4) (status 20))
 (segment (start 263.5 94.625) (end 263.5 92.5) (width 1) (layer B.Cu) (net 4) (status 10))
 (segment (start 264.75 91.25) (end 270.25 91.25) (width 1) (layer B.Cu) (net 4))
 (segment (start 263.5 92.5) (end 264.75 91.25) (width 1) (layer B.Cu) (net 4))
 (segment (start 270.25 88.1) (end 270.25 91.25) (width 1) (layer B.Cu) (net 4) (status 10))
 (segment (start 270.25 91.25) (end 270.25 94.4) (width 1) (layer B.Cu) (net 4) (status 20))
 (segment (start 25 28.75) (end 25 27.25) (width 0.25) (layer F.Cu) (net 5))
 (segment (start 25 27.25) (end 26 27.25) (width 0.25) (layer +5V) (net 5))
 (via (at 25 27.25) (size 0.6) (drill 0.4) (layers F.Cu B.Cu) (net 5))
 (segment (start 29.5 27.9) (end 25.85 27.9) (width 0.25) (layer F.Cu) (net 5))
 (segment (start 25.85 27.9) (end 25 28.75) (width 0.25) (layer F.Cu) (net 5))
 (segment (start 266.25 110.5) (end 266.25 102.125) (width 1) (layer B.Cu) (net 5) (status 10))
 (via (at 266.25 102.125) (size 0.6) (drill 0.4) (layers F.Cu B.Cu) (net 5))
 (segment (start 266.25 102.125) (end 266.25 102.25) (width 1) (layer +5V) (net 5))
 (segment (start 268.875 99.5) (end 268.875 97.875) (width 1) (layer B.Cu) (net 5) (status 10))
 (segment (start 267.95 96.95) (end 267.95 94.4) (width 1) (layer B.Cu) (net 5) (status 20))
 (segment (start 268.875 97.875) (end 267.95 96.95) (width 1) (layer B.Cu) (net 5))
 (segment (start 266.25 102.125) (end 268.875 99.5) (width 1) (layer B.Cu) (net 5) (status 20))
 (segment (start 270.5 125.04986) (end 270.5 114.75) (width 1) (layer B.Cu) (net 5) (status 10))
 (segment (start 270.5 114.75) (end 266.25 110.5) (width 1) (layer B.Cu) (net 5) (status 20))
 (segment (start 250.25 96.55) (end 246.59986 96.55) (width 0.25) (layer B.Cu) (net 6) (status 30))
 (segment (start 246.59986 96.55) (end 246.59982 96.55004) (width 0.25) (layer B.Cu) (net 6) (status 30))
 (segment (start 246.75 93.5) (end 246.75 96.39986) (width 0.25) (layer B.Cu) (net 6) (status 30))
 (segment (start 246.75 96.39986) (end 246.90014 96.55) (width 0.25) (layer B.Cu) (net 6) (status 30))
 (segment (start 246.90014 96.55) (end 258.25 96.55) (width 0.25) (layer B.Cu) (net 6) (status 30))
 (segment (start 240.4 105.75) (end 239.25 105.75) (width 0.25) (layer B.Cu) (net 8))
 (segment (start 36.6 27.9) (end 34.5 27.9) (width 0.25) (layer F.Cu) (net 8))
 (segment (start 36.75 27.75) (end 36.6 27.9) (width 0.25) (layer F.Cu) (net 8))
 (via (at 36.75 27.75) (size 0.6) (drill 0.4) (layers F.Cu B.Cu) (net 8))
 (segment (start 161.25 27.75) (end 36.75 27.75) (width 0.25) (layer B.Cu) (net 8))
 (segment (start 233.5 100) (end 161.25 27.75) (width 0.25) (layer B.Cu) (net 8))
 (segment (start 233.5 104.25) (end 233.5 100) (width 0.25) (layer B.Cu) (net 8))
 (via (at 233.5 104.25) (size 0.6) (drill 0.4) (layers F.Cu B.Cu) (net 8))
 (segment (start 236 104.25) (end 233.5 104.25) (width 0.25) (layer F.Cu) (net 8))
 (via (at 236 104.25) (size 0.6) (drill 0.4) (layers F.Cu B.Cu) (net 8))
 (segment (start 237.75 104.25) (end 236 104.25) (width 0.25) (layer B.Cu) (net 8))
 (segment (start 239.25 105.75) (end 237.75 104.25) (width 0.25) (layer B.Cu) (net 8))
 (segment (start 257 106.75) (end 256 107.75) (width 0.25) (layer B.Cu) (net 9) (status 10))
 (segment (start 256 107.75) (end 249.1 107.75) (width 0.25) (layer B.Cu) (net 9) (status 20))
 (segment (start 257 109.29) (end 255.96 108.25) (width 0.25) (layer B.Cu) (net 10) (status 10))
 (segment (start 255.96 108.25) (end 249.1 108.25) (width 0.25) (layer B.Cu) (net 10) (status 20))
 (segment (start 244 112.35) (end 244 116.25) (width 0.25) (layer B.Cu) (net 11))
 (segment (start 244 117.75) (end 244 120) (width 0.25) (layer B.Cu) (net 12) (status 30))
 (segment (start 250.25 117.8) (end 244.05 117.8) (width 0.25) (layer B.Cu) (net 12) (status 30))
 (segment (start 244.05 117.8) (end 244 117.75) (width 0.25) (layer B.Cu) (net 12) (status 30))
 (segment (start 258.25 117.8) (end 250.25 117.8) (width 0.25) (layer B.Cu) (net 12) (status 30))
 (segment (start 240.4 107.75) (end 241.75 107.75) (width 0.25) (layer B.Cu) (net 16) (status 10))
 (segment (start 241.44996 96.55004) (end 244.40018 96.55004) (width 0.25) (layer B.Cu) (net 16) (status 20))
 (segment (start 240.5 97.5) (end 241.44996 96.55004) (width 0.25) (layer B.Cu) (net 16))
 (segment (start 240.5 103.75) (end 240.5 97.5) (width 0.25) (layer B.Cu) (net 16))
 (segment (start 242.25 105.5) (end 240.5 103.75) (width 0.25) (layer B.Cu) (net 16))
 (segment (start 242.25 107.25) (end 242.25 105.5) (width 0.25) (layer B.Cu) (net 16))
 (segment (start 241.75 107.75) (end 242.25 107.25) (width 0.25) (layer B.Cu) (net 16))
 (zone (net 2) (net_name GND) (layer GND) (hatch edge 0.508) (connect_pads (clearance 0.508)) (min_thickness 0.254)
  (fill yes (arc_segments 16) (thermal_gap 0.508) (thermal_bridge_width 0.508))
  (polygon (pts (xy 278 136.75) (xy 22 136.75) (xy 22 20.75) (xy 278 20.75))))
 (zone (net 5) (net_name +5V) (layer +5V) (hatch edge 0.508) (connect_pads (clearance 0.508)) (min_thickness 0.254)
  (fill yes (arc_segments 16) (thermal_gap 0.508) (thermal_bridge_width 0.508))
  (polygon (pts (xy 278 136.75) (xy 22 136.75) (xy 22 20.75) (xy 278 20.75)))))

